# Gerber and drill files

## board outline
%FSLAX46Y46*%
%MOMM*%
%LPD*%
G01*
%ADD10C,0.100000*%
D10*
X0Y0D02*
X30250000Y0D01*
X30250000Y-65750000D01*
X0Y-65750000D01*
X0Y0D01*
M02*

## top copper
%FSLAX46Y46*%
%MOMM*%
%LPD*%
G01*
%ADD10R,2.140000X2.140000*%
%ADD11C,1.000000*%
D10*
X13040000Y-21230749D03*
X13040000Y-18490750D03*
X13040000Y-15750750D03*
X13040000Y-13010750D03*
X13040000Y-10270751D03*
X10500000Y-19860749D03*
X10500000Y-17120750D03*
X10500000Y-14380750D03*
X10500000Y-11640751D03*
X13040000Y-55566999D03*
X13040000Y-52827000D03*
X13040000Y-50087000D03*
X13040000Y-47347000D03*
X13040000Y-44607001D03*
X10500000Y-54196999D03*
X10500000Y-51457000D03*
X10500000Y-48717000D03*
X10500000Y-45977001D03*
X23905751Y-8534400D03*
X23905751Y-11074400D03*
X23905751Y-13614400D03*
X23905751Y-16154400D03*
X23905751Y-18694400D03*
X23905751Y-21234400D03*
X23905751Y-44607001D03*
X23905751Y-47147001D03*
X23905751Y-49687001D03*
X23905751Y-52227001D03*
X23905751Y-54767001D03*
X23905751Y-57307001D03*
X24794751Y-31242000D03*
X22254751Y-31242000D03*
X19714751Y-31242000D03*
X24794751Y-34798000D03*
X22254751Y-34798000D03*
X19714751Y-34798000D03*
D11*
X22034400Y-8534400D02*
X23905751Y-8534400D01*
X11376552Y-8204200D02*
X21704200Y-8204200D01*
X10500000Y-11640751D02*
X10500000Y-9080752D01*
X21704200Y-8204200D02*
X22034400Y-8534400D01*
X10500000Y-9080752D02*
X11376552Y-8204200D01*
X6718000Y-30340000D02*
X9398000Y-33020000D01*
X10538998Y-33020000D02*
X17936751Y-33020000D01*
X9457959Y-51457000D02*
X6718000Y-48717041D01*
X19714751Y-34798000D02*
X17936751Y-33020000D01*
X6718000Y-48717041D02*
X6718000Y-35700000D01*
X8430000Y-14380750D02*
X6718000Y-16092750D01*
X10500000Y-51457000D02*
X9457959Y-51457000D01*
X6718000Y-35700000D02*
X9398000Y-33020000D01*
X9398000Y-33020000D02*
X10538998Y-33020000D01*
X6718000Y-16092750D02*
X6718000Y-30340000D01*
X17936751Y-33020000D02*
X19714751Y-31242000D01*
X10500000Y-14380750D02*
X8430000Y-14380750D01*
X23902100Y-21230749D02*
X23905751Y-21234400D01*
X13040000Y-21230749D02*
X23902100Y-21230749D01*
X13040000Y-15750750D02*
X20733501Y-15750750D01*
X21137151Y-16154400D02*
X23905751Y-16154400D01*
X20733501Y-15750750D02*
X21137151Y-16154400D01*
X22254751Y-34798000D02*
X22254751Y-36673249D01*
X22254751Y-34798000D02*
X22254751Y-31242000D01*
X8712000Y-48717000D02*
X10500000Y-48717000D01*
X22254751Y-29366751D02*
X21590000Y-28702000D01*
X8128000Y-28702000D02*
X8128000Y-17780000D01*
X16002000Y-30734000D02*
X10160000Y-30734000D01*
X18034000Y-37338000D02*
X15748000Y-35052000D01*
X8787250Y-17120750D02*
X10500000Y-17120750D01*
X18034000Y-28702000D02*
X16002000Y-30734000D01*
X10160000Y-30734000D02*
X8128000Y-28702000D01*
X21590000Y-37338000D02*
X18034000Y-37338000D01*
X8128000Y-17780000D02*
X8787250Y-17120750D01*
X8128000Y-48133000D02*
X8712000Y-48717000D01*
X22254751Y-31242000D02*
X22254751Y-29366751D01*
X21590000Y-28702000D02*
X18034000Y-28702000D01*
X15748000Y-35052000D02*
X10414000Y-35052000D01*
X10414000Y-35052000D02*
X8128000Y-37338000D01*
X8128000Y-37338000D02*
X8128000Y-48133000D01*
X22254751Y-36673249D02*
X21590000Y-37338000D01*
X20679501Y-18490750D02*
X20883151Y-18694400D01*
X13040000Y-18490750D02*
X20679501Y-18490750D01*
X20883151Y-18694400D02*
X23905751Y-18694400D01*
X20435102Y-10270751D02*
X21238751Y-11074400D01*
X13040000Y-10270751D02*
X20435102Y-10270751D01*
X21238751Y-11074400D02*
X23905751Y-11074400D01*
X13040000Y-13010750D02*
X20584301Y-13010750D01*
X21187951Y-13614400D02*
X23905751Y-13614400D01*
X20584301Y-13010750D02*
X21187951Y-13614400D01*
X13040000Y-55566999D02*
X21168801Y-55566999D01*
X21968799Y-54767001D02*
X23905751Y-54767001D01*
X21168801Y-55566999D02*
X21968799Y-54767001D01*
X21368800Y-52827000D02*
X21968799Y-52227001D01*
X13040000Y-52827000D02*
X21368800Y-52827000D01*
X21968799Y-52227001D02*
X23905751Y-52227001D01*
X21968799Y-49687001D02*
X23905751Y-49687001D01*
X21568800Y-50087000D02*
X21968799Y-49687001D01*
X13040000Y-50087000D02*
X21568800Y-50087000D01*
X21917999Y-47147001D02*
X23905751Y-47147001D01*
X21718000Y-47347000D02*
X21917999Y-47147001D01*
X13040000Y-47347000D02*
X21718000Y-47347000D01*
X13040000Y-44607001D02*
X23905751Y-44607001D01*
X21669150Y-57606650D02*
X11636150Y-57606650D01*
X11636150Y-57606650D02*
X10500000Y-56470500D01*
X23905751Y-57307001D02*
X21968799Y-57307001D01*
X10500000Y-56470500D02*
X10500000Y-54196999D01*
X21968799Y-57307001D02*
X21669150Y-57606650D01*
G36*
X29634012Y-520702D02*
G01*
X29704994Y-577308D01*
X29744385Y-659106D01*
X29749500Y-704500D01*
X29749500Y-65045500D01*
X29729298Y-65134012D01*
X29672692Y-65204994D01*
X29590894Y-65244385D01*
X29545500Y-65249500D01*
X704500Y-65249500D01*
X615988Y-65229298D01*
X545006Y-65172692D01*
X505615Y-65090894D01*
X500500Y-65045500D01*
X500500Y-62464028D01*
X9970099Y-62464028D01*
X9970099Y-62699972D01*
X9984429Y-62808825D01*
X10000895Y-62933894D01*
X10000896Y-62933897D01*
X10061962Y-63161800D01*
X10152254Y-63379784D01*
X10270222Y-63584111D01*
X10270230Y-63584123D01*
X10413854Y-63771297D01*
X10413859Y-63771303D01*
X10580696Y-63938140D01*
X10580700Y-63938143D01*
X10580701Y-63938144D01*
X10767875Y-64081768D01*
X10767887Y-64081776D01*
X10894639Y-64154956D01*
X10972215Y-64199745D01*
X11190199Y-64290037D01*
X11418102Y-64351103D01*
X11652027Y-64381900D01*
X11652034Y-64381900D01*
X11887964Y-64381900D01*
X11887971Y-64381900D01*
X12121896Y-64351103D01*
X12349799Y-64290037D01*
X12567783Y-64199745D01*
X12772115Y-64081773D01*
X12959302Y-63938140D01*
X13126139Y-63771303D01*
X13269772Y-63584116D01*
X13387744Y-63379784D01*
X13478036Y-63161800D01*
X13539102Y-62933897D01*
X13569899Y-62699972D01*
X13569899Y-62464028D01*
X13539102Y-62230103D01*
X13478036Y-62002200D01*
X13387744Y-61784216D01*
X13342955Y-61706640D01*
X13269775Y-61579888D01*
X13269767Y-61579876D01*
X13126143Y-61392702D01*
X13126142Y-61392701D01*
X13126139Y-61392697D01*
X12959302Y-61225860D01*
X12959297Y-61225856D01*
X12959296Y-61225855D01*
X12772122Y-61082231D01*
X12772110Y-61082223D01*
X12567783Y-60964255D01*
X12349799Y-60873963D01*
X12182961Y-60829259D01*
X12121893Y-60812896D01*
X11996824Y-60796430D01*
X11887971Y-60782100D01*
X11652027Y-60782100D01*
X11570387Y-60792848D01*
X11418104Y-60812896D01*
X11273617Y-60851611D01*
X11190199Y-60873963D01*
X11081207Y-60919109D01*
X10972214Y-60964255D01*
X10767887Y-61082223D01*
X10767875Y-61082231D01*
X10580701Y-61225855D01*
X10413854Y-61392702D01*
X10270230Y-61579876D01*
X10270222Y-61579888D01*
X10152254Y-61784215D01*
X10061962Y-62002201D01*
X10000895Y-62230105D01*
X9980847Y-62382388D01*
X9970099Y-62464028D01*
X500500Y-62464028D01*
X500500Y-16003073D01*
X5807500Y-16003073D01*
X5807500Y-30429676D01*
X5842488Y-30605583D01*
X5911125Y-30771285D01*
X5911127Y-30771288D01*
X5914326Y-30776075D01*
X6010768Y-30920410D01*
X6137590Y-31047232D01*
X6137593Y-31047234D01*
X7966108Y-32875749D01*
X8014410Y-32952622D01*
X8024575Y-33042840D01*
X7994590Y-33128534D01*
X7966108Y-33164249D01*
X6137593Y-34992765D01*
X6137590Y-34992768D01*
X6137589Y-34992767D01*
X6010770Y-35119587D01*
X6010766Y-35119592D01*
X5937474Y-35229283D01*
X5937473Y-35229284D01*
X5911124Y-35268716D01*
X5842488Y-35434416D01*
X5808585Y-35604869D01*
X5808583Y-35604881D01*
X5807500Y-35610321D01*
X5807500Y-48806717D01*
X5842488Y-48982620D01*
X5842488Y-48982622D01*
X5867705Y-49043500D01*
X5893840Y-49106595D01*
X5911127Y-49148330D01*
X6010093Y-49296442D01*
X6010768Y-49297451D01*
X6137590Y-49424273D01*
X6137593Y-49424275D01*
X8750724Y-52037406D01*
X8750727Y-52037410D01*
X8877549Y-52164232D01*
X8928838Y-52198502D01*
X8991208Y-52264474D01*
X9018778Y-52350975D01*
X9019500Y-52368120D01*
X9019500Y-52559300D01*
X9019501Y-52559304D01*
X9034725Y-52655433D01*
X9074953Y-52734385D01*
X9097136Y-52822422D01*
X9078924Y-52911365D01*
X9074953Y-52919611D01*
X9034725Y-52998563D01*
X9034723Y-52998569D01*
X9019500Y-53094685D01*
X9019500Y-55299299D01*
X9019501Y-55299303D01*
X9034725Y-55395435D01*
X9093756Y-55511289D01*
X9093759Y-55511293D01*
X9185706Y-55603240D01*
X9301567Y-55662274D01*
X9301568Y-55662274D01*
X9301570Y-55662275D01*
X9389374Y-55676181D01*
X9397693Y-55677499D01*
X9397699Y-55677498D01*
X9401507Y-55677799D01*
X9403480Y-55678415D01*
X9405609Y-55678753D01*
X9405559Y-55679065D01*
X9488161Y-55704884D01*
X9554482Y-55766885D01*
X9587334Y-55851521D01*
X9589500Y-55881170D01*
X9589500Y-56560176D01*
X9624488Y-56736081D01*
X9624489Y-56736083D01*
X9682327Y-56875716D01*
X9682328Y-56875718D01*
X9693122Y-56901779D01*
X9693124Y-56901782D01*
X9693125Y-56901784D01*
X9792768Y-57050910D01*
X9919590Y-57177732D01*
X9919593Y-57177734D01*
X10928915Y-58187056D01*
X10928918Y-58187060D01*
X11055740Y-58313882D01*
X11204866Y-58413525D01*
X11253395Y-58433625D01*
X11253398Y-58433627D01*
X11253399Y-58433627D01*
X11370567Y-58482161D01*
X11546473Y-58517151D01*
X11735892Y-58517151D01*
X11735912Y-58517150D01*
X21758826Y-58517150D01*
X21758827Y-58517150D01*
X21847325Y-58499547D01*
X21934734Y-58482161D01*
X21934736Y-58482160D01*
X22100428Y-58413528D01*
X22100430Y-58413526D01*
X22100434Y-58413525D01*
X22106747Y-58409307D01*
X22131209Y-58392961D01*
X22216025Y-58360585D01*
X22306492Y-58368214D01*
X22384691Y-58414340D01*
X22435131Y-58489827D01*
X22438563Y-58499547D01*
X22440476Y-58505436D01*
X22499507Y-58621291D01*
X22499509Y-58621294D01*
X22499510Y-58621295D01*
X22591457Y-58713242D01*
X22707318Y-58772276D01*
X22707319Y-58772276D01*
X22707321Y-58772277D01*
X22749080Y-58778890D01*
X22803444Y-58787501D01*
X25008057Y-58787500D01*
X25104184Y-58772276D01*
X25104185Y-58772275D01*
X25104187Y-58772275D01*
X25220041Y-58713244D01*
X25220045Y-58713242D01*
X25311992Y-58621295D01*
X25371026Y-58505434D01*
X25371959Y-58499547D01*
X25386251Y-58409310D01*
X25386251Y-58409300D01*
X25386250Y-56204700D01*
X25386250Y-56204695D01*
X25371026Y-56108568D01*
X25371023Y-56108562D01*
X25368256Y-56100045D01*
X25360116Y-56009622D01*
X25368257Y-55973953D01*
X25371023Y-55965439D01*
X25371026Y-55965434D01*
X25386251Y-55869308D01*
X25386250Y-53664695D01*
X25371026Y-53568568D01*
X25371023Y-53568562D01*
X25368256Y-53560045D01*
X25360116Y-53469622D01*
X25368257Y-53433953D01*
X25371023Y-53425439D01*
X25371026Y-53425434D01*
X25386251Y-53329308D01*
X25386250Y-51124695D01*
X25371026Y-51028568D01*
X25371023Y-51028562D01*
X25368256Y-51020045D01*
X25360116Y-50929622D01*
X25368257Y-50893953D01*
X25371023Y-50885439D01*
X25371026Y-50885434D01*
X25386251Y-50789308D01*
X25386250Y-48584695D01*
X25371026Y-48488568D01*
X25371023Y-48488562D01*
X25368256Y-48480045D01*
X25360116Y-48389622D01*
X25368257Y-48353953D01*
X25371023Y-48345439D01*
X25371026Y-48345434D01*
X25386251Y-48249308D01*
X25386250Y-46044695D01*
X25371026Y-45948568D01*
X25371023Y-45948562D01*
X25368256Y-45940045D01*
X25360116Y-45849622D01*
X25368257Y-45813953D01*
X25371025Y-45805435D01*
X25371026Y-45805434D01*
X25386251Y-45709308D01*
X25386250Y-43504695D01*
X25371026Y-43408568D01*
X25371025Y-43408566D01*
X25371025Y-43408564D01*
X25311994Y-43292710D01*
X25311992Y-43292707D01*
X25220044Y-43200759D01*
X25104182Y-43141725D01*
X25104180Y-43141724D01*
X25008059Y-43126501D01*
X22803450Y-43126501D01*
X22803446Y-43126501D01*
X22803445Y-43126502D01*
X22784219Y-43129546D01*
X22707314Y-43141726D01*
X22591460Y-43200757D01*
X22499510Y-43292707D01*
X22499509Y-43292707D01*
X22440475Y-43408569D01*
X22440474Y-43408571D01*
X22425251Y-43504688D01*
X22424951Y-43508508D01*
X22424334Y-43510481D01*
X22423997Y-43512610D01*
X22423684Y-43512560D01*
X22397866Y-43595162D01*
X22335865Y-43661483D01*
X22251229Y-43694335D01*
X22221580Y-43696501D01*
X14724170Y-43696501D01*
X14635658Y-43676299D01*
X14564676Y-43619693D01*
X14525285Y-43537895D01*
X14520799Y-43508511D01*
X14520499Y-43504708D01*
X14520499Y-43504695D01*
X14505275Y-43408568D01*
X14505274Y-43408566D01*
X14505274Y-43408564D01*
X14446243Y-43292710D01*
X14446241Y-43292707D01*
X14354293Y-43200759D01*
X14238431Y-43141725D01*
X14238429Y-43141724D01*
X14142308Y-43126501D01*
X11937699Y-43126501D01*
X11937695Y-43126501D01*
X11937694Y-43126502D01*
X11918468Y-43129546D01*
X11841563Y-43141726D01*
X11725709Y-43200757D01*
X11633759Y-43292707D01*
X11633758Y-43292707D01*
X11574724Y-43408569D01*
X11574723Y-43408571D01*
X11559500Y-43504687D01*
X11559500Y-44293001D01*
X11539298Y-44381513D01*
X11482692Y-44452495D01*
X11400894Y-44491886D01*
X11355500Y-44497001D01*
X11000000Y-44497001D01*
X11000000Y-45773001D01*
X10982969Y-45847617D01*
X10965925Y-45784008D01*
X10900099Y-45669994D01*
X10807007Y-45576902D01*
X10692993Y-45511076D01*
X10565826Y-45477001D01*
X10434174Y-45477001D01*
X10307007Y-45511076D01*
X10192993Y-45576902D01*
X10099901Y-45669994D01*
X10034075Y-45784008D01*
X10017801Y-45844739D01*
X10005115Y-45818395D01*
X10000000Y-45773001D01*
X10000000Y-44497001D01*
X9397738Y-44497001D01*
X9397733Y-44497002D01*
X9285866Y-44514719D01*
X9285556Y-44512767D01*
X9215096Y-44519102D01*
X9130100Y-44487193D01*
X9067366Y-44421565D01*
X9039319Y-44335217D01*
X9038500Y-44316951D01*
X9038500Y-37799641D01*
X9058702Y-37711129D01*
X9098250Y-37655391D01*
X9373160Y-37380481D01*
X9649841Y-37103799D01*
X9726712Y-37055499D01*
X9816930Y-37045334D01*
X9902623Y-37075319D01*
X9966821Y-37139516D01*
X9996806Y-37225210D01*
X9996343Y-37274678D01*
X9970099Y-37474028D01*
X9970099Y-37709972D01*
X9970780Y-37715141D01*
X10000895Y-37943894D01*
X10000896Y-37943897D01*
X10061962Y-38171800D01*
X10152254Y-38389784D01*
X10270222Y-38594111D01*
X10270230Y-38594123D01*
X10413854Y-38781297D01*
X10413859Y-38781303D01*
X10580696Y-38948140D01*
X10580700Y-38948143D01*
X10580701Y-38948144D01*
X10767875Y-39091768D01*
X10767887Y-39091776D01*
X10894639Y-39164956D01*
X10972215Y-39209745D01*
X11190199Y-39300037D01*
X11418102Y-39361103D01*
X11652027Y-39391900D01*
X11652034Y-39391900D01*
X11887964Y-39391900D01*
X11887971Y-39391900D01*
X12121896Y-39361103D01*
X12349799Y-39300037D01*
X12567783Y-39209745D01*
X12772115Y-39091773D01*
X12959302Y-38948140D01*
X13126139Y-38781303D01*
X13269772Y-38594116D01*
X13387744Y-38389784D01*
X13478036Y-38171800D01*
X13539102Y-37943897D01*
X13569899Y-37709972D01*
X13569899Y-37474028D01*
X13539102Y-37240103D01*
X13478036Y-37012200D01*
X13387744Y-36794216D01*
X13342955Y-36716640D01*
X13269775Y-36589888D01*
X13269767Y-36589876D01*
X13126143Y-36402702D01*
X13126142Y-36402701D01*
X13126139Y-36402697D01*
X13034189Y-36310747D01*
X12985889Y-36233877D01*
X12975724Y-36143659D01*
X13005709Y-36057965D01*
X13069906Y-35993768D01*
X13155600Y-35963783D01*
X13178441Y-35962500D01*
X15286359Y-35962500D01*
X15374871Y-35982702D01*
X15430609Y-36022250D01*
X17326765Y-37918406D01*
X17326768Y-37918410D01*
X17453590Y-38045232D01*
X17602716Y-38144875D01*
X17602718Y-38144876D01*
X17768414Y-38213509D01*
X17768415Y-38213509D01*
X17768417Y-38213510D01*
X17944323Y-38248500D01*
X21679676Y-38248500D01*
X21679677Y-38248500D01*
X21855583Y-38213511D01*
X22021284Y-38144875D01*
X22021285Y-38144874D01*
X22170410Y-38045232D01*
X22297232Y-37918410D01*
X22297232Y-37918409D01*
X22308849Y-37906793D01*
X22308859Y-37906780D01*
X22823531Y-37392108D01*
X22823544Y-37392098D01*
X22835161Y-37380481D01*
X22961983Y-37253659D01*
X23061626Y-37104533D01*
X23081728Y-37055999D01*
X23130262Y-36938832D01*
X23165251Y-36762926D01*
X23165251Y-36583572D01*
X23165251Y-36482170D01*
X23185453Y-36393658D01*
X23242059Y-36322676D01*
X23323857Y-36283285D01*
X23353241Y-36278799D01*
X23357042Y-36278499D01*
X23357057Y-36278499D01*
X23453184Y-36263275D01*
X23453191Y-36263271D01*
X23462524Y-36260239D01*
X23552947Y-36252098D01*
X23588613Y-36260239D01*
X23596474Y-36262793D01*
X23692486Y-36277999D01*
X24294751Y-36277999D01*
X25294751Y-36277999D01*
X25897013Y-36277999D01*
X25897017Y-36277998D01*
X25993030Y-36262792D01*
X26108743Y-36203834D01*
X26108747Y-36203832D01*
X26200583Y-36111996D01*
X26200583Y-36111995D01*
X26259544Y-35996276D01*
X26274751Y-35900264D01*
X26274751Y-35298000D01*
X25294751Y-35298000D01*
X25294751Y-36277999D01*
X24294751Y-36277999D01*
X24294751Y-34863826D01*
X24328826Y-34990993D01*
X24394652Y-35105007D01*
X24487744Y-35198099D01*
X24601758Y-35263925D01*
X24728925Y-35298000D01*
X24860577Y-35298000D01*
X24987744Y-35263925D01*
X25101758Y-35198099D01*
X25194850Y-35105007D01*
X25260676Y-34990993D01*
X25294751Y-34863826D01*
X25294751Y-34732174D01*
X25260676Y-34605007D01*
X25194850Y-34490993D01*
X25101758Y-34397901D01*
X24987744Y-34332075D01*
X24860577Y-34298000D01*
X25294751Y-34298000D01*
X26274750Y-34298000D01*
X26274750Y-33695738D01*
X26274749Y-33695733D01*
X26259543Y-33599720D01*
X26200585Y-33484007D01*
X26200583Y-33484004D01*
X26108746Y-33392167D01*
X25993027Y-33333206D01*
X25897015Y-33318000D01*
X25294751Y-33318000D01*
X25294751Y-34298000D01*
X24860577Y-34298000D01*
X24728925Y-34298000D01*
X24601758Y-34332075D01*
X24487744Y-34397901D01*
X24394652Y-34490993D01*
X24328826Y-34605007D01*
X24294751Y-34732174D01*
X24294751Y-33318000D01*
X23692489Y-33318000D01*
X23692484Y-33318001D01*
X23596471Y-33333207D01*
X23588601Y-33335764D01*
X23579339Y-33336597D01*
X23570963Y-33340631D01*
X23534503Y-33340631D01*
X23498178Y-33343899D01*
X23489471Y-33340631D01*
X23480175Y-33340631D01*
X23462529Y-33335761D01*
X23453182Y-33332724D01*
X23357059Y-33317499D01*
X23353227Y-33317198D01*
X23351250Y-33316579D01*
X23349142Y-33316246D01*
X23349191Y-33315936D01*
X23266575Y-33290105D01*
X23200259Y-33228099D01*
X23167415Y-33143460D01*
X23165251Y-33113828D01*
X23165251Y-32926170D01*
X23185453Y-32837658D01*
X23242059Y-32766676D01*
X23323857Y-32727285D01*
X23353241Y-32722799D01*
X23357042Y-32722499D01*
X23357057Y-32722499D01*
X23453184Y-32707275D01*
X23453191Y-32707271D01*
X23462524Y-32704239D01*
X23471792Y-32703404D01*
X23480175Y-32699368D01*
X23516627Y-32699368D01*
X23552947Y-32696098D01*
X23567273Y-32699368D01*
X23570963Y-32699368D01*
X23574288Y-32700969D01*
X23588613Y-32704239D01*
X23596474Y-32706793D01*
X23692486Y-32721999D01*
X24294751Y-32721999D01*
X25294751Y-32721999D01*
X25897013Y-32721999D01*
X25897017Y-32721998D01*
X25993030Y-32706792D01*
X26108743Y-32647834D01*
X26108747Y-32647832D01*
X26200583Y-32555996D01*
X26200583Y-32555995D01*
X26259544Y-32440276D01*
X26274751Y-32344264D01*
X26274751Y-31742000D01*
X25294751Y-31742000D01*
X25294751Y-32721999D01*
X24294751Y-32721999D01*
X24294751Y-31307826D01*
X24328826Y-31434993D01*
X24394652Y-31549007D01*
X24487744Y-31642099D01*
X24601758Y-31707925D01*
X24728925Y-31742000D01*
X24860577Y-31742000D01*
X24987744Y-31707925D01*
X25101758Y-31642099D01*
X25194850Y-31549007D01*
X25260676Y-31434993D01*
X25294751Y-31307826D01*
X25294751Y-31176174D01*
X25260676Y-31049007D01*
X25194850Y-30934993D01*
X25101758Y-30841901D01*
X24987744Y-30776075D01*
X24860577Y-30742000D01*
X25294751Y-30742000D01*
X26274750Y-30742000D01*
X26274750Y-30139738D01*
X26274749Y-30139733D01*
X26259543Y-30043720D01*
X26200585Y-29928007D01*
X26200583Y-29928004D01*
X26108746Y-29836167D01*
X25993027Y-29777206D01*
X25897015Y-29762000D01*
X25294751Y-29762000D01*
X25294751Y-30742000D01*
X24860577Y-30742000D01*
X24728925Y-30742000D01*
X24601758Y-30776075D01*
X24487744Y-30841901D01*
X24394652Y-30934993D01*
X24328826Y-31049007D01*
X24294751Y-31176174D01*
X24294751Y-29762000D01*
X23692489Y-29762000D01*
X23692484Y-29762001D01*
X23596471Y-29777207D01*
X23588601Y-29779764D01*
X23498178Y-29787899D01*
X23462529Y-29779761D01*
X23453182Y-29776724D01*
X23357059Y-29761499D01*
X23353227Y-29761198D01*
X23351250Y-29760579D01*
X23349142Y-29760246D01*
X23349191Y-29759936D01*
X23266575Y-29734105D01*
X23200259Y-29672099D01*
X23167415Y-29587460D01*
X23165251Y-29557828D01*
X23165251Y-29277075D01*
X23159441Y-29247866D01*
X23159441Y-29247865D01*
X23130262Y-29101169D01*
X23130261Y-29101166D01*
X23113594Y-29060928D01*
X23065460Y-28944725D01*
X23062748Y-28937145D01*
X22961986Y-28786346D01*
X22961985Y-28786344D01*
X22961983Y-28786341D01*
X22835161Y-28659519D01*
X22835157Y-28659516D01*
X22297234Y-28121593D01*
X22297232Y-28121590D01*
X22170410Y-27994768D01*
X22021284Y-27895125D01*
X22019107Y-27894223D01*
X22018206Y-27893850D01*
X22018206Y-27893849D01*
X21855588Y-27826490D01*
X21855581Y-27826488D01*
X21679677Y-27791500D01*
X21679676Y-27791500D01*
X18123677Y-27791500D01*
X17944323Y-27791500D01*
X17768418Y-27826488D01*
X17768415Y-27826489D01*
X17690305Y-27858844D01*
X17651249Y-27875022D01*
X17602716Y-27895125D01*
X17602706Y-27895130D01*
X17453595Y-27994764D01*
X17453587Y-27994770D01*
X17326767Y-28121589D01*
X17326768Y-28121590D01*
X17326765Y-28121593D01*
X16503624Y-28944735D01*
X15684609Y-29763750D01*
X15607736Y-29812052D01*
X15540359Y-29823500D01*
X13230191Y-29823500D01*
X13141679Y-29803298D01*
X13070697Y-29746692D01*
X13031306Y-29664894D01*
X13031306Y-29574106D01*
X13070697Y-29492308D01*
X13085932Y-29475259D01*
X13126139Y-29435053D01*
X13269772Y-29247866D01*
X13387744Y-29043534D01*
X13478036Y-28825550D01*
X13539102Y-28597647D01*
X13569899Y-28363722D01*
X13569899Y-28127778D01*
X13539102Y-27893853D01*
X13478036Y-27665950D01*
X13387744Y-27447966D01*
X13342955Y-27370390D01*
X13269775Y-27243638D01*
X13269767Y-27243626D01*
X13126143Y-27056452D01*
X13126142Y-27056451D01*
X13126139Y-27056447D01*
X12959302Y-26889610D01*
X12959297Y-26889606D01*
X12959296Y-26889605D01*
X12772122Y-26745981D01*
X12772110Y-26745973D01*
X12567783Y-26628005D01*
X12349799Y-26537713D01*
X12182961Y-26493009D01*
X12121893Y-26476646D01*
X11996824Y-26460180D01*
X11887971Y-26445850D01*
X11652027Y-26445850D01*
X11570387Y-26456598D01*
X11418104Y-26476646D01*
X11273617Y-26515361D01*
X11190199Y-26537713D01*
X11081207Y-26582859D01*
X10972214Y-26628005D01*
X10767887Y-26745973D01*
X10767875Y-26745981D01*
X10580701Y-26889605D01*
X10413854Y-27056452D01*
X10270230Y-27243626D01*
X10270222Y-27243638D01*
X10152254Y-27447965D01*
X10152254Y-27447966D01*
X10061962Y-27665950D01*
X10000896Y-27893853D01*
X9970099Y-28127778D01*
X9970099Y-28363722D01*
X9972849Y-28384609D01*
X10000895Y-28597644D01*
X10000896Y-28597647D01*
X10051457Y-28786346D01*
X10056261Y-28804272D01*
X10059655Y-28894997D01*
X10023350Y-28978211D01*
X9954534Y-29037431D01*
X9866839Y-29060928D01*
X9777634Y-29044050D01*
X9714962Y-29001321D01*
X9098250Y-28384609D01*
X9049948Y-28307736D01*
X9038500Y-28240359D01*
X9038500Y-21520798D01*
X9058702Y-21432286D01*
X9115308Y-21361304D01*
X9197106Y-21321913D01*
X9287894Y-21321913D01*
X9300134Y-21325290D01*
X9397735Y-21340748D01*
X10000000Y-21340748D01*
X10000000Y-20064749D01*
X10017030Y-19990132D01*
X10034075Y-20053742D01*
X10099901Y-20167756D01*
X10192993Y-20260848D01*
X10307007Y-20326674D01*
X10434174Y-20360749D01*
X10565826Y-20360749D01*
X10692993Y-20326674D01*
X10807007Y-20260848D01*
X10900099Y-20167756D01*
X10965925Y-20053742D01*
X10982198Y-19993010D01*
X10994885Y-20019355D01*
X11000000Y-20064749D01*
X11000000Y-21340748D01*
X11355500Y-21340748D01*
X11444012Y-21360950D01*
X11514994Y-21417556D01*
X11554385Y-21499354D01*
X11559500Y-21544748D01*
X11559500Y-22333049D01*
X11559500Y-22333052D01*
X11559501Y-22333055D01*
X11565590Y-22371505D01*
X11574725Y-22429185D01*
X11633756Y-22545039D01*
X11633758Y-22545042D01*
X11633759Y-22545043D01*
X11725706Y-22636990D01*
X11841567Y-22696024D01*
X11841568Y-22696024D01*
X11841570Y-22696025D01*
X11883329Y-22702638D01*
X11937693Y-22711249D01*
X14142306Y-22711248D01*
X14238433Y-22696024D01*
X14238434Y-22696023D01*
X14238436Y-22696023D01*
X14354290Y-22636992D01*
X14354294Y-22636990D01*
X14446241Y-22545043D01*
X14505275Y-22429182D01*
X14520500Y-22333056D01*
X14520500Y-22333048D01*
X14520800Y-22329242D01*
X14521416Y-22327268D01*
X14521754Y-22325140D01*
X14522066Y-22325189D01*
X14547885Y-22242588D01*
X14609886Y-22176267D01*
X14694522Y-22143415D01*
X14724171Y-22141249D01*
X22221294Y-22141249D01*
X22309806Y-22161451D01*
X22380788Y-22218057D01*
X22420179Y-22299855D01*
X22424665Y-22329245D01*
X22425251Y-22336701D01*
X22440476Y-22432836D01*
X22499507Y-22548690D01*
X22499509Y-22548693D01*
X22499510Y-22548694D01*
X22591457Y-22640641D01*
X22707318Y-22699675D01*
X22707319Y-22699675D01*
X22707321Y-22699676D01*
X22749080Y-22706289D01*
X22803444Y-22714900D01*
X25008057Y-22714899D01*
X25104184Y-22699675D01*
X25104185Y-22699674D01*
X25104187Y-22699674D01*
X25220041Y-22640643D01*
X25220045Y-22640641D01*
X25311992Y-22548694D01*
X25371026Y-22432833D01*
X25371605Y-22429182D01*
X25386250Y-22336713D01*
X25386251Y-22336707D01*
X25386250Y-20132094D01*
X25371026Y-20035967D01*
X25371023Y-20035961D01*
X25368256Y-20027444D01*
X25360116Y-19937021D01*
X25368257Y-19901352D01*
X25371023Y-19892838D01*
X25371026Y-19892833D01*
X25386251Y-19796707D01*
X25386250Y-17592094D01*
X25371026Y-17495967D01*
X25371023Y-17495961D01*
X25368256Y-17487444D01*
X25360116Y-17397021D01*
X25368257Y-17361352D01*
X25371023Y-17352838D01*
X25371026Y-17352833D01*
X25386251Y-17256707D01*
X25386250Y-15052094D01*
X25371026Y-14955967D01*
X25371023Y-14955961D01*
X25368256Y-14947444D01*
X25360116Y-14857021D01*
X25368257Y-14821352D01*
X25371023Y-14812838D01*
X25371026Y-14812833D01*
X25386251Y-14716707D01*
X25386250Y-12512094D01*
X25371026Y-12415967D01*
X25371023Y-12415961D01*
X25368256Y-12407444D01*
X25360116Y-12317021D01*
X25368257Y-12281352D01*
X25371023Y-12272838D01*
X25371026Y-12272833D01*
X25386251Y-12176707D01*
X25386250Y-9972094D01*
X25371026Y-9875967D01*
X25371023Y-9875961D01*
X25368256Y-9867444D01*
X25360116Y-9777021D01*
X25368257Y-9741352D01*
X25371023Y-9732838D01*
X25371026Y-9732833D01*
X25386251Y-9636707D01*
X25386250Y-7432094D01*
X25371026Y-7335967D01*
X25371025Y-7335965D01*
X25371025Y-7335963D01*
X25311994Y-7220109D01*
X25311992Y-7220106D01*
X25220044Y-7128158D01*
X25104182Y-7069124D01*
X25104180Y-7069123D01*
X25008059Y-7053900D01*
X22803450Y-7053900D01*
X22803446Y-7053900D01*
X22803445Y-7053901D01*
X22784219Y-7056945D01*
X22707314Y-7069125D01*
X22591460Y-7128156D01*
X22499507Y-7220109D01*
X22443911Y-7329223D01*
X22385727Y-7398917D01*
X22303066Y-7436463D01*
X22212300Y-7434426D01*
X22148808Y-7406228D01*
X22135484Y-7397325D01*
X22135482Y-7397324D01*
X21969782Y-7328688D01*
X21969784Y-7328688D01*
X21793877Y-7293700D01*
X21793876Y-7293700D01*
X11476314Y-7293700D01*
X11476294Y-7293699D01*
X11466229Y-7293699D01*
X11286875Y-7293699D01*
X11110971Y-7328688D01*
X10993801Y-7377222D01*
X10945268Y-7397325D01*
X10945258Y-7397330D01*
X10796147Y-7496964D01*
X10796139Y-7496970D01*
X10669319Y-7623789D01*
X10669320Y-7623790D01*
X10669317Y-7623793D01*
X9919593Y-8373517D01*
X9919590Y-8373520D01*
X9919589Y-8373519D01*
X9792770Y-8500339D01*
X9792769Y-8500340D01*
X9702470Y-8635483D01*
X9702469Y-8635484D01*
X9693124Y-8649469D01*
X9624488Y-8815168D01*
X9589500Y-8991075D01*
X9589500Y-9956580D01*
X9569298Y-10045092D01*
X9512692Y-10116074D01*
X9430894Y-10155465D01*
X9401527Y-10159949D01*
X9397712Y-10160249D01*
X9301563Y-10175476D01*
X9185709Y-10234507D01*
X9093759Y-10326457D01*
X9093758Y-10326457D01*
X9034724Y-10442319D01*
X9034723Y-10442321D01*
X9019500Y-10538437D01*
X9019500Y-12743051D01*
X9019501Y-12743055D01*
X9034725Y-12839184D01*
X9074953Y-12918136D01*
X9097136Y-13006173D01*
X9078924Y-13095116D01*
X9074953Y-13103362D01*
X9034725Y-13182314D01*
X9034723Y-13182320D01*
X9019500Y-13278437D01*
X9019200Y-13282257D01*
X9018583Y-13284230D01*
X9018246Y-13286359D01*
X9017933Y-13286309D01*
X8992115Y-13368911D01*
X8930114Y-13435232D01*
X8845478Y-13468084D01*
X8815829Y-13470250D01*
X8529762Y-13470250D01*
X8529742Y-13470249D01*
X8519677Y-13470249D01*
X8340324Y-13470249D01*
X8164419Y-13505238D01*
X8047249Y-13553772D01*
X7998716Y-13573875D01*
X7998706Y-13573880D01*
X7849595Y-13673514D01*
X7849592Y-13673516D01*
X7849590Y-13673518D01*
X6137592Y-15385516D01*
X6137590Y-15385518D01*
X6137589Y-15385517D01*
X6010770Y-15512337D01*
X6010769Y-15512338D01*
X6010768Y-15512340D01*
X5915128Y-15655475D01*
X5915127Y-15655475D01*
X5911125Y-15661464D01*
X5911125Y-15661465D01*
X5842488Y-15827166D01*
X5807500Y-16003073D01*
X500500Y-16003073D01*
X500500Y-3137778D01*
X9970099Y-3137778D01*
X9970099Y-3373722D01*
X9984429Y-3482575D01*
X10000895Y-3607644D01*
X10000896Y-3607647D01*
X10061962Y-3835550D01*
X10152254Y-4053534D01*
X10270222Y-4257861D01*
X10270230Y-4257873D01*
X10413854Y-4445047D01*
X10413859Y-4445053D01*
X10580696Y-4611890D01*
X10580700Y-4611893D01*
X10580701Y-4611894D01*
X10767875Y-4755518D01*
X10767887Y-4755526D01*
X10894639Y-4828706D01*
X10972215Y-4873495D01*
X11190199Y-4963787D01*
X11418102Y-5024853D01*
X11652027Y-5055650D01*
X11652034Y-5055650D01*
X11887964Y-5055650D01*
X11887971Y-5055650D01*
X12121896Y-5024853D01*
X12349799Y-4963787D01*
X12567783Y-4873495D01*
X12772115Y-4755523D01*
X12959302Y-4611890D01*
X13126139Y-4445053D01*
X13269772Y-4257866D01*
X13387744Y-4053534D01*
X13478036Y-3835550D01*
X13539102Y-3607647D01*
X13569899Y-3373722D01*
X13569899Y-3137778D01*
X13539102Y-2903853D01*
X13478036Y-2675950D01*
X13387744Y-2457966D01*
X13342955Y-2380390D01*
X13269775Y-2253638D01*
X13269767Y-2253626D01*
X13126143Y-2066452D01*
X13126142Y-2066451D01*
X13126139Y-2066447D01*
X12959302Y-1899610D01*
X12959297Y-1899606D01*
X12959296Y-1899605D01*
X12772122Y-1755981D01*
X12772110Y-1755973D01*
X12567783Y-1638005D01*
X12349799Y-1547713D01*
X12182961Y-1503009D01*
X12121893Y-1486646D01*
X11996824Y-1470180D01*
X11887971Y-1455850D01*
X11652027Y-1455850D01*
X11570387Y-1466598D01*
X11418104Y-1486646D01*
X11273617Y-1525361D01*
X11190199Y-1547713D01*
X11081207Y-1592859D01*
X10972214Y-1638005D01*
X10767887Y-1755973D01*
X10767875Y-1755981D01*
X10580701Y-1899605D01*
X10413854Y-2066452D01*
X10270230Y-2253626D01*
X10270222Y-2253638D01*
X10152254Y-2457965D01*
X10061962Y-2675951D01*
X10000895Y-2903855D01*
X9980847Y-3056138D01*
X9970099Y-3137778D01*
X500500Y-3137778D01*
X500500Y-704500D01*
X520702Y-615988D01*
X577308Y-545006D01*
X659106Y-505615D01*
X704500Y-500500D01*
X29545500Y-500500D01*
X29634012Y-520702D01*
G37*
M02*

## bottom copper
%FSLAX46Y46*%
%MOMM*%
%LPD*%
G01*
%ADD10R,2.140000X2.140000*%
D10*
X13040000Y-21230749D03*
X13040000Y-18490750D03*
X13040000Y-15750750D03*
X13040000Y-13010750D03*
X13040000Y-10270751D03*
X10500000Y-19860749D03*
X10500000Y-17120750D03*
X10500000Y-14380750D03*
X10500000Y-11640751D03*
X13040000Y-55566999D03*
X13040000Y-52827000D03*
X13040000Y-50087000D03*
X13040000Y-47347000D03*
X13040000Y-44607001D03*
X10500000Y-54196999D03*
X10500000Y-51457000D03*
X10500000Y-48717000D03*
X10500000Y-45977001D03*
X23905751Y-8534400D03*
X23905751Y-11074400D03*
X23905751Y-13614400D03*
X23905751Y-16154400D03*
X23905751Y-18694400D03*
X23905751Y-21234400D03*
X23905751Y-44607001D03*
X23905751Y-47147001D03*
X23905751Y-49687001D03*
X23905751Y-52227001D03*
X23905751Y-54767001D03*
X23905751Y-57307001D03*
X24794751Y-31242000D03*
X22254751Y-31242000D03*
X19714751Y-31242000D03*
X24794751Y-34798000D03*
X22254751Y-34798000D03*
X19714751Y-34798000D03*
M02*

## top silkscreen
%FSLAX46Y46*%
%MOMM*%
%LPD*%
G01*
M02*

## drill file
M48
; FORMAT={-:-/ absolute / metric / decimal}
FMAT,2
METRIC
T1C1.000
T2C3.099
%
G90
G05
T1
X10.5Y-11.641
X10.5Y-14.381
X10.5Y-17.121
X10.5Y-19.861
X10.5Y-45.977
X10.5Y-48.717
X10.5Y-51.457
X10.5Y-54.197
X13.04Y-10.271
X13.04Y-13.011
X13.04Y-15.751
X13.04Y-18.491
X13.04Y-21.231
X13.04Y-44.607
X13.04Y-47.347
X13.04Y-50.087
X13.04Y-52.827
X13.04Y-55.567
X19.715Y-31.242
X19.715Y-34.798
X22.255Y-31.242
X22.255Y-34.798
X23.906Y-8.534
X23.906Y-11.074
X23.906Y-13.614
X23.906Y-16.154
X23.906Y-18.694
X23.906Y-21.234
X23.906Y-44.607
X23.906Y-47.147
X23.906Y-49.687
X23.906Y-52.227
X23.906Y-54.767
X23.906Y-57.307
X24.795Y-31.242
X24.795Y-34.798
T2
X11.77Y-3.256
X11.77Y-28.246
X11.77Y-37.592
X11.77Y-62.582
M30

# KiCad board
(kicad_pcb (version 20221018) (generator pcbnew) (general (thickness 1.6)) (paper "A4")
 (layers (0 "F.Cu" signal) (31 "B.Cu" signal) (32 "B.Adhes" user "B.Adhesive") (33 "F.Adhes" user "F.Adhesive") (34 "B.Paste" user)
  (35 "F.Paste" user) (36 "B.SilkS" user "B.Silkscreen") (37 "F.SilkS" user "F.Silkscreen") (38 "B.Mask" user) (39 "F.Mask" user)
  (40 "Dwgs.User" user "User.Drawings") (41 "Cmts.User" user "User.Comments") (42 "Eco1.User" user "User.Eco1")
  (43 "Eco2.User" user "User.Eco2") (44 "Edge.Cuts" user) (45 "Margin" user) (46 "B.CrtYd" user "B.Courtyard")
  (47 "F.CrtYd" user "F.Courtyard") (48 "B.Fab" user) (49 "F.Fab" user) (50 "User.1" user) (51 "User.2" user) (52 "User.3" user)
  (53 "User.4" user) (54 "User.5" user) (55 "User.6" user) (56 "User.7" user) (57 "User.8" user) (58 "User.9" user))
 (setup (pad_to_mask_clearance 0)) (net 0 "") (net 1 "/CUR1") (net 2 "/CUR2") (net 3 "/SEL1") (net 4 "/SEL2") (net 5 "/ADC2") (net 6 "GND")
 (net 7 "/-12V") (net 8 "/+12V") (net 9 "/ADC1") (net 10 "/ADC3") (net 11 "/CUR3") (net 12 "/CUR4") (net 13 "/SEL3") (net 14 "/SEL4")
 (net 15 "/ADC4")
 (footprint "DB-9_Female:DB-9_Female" (layer "B.Cu") (at 0.1 15.75075 -90)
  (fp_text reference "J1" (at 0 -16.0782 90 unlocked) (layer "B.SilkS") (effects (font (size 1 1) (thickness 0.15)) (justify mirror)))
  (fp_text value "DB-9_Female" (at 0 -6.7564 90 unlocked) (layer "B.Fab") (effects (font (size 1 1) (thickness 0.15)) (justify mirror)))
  (pad "" np_thru_hole circle (at -12.495 -11.669999 270) (size 3.0988 3.0988) (drill 3.0988) (layers "*.Cu" "*.Mask"))
  (pad "" np_thru_hole circle (at 12.495 -11.669999 270) (size 3.0988 3.0988) (drill 3.0988) (layers "*.Cu" "*.Mask"))
  (pad "1" thru_hole rect (at 5.479999 -12.94 270) (size 2.14 2.14) (drill 1) (layers "*.Cu" "*.Mask") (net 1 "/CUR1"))
  (pad "2" thru_hole rect (at 2.74 -12.94 270) (size 2.14 2.14) (drill 1) (layers "*.Cu" "*.Mask") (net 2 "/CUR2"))
  (pad "3" thru_hole rect (at 0 -12.94 270) (size 2.14 2.14) (drill 1) (layers "*.Cu" "*.Mask") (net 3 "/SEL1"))
  (pad "4" thru_hole rect (at -2.74 -12.94 270) (size 2.14 2.14) (drill 1) (layers "*.Cu" "*.Mask") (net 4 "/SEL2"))
  (pad "5" thru_hole rect (at -5.479999 -12.94 270) (size 2.14 2.14) (drill 1) (layers "*.Cu" "*.Mask") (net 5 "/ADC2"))
  (pad "6" thru_hole rect (at 4.109999 -10.4 270) (size 2.14 2.14) (drill 1) (layers "*.Cu" "*.Mask") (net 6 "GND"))
  (pad "7" thru_hole rect (at 1.37 -10.4 270) (size 2.14 2.14) (drill 1) (layers "*.Cu" "*.Mask") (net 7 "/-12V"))
  (pad "8" thru_hole rect (at -1.37 -10.4 270) (size 2.14 2.14) (drill 1) (layers "*.Cu" "*.Mask") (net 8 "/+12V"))
  (pad "9" thru_hole rect (at -4.109999 -10.4 270) (size 2.14 2.14) (drill 1) (layers "*.Cu" "*.Mask") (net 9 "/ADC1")))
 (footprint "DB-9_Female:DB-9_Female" (layer "B.Cu") (at 0.1 50.087 -90)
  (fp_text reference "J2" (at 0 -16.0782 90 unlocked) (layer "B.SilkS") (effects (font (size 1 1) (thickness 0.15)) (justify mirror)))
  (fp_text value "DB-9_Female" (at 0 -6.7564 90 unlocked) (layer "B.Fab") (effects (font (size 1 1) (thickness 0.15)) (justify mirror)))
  (pad "" np_thru_hole circle (at -12.495 -11.669999 270) (size 3.0988 3.0988) (drill 3.0988) (layers "*.Cu" "*.Mask"))
  (pad "" np_thru_hole circle (at 12.495 -11.669999 270) (size 3.0988 3.0988) (drill 3.0988) (layers "F&B.Cu" "*.Mask"))
  (pad "1" thru_hole rect (at 5.479999 -12.94 270) (size 2.14 2.14) (drill 1) (layers "*.Cu" "*.Mask") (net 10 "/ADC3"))
  (pad "2" thru_hole rect (at 2.74 -12.94 270) (size 2.14 2.14) (drill 1) (layers "*.Cu" "*.Mask") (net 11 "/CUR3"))
  (pad "3" thru_hole rect (at 0 -12.94 270) (size 2.14 2.14) (drill 1) (layers "*.Cu" "*.Mask") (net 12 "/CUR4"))
  (pad "4" thru_hole rect (at -2.74 -12.94 270) (size 2.14 2.14) (drill 1) (layers "*.Cu" "*.Mask") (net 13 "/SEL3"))
  (pad "5" thru_hole rect (at -5.479999 -12.94 270) (size 2.14 2.14) (drill 1) (layers "*.Cu" "*.Mask") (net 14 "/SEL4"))
  (pad "6" thru_hole rect (at 4.109999 -10.4 270) (size 2.14 2.14) (drill 1) (layers "*.Cu" "*.Mask") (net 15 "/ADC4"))
  (pad "7" thru_hole rect (at 1.37 -10.4 270) (size 2.14 2.14) (drill 1) (layers "*.Cu" "*.Mask") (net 8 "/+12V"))
  (pad "8" thru_hole rect (at -1.37 -10.4 270) (size 2.14 2.14) (drill 1) (layers "*.Cu" "*.Mask") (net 7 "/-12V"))
  (pad "9" thru_hole rect (at -4.109999 -10.4 270) (size 2.14 2.14) (drill 1) (layers "*.Cu" "*.Mask") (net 6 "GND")))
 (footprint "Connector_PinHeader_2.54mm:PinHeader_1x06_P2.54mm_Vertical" (layer "B.Cu") (at 23.905751 8.5344 180)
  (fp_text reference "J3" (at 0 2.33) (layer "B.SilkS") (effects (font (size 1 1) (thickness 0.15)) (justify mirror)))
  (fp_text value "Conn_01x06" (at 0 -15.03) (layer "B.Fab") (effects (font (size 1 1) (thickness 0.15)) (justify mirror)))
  (pad "1" thru_hole rect (at 0 0 180) (size 2.14 2.14) (drill 1) (layers "*.Cu" "*.Mask") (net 9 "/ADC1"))
  (pad "2" thru_hole rect (at 0 -2.54 180) (size 2.14 2.14) (drill 1) (layers "*.Cu" "*.Mask") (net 5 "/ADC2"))
  (pad "3" thru_hole rect (at 0 -5.08 180) (size 2.14 2.14) (drill 1) (layers "*.Cu" "*.Mask") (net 4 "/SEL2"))
  (pad "4" thru_hole rect (at 0 -7.62 180) (size 2.14 2.14) (drill 1) (layers "*.Cu" "*.Mask") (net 3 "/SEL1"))
  (pad "5" thru_hole rect (at 0 -10.16 180) (size 2.14 2.14) (drill 1) (layers "*.Cu" "*.Mask") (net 2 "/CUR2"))
  (pad "6" thru_hole rect (at 0 -12.7 180) (size 2.14 2.14) (drill 1) (layers "*.Cu" "*.Mask") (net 1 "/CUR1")))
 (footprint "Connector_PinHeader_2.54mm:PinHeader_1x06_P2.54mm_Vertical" (layer "B.Cu") (at 23.905751 44.607001 180)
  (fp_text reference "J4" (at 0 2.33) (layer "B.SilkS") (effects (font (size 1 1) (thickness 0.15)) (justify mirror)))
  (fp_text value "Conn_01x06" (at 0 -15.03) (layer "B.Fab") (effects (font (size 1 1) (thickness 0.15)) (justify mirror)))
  (pad "1" thru_hole rect (at 0 0 180) (size 2.14 2.14) (drill 1) (layers "*.Cu" "*.Mask") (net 14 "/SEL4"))
  (pad "2" thru_hole rect (at 0 -2.54 180) (size 2.14 2.14) (drill 1) (layers "*.Cu" "*.Mask") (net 13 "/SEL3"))
  (pad "3" thru_hole rect (at 0 -5.08 180) (size 2.14 2.14) (drill 1) (layers "*.Cu" "*.Mask") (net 12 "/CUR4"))
  (pad "4" thru_hole rect (at 0 -7.62 180) (size 2.14 2.14) (drill 1) (layers "*.Cu" "*.Mask") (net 11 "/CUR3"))
  (pad "5" thru_hole rect (at 0 -10.16 180) (size 2.14 2.14) (drill 1) (layers "*.Cu" "*.Mask") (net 10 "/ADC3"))
  (pad "6" thru_hole rect (at 0 -12.7 180) (size 2.14 2.14) (drill 1) (layers "*.Cu" "*.Mask") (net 15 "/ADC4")))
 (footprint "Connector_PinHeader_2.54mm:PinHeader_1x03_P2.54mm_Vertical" (layer "B.Cu") (at 24.794751 31.242 90)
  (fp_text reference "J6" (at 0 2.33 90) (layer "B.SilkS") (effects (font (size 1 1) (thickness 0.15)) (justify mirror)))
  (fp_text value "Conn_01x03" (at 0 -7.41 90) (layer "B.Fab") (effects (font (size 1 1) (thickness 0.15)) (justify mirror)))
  (pad "1" thru_hole rect (at 0 0 90) (size 2.14 2.14) (drill 1) (layers "*.Cu" "*.Mask") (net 6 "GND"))
  (pad "2" thru_hole rect (at 0 -2.54 90) (size 2.14 2.14) (drill 1) (layers "*.Cu" "*.Mask") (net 7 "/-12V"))
  (pad "3" thru_hole rect (at 0 -5.08 90) (size 2.14 2.14) (drill 1) (layers "*.Cu" "*.Mask") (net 8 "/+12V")))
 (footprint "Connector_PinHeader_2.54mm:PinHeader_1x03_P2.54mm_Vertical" (layer "B.Cu") (at 24.794751 34.798 90)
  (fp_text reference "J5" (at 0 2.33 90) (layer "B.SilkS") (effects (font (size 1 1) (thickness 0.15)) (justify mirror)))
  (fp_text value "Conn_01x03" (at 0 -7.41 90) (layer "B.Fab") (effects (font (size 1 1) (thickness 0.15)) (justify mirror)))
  (pad "1" thru_hole rect (at 0 0 90) (size 2.14 2.14) (drill 1) (layers "*.Cu" "*.Mask") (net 6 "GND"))
  (pad "2" thru_hole rect (at 0 -2.54 90) (size 2.14 2.14) (drill 1) (layers "*.Cu" "*.Mask") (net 7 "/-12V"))
  (pad "3" thru_hole rect (at 0 -5.08 90) (size 2.14 2.14) (drill 1) (layers "*.Cu" "*.Mask") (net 8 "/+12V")))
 (gr_rect (start 0 0) (end 30.25 65.75) (stroke (width 0.1) (type default)) (fill none) (layer "Edge.Cuts"))
 (segment (start 22.0344 8.5344) (end 23.905751 8.5344) (width 1) (layer "F.Cu") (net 9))
 (segment (start 11.376552 8.2042) (end 21.7042 8.2042) (width 1) (layer "F.Cu") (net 9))
 (segment (start 10.5 11.640751) (end 10.5 9.080752) (width 1) (layer "F.Cu") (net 9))
 (segment (start 21.7042 8.2042) (end 22.0344 8.5344) (width 1) (layer "F.Cu") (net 9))
 (segment (start 10.5 9.080752) (end 11.376552 8.2042) (width 1) (layer "F.Cu") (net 9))
 (segment (start 6.718 30.34) (end 9.398 33.02) (width 1) (layer "F.Cu") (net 8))
 (segment (start 10.538998 33.02) (end 17.936751 33.02) (width 1) (layer "F.Cu") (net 8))
 (segment (start 9.457959 51.457) (end 6.718 48.717041) (width 1) (layer "F.Cu") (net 8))
 (segment (start 19.714751 34.798) (end 17.936751 33.02) (width 1) (layer "F.Cu") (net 8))
 (segment (start 6.718 48.717041) (end 6.718 35.7) (width 1) (layer "F.Cu") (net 8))
 (segment (start 8.43 14.38075) (end 6.718 16.09275) (width 1) (layer "F.Cu") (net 8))
 (segment (start 10.5 51.457) (end 9.457959 51.457) (width 1) (layer "F.Cu") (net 8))
 (segment (start 6.718 35.7) (end 9.398 33.02) (width 1) (layer "F.Cu") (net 8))
 (segment (start 9.398 33.02) (end 10.538998 33.02) (width 1) (layer "F.Cu") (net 8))
 (segment (start 6.718 16.09275) (end 6.718 30.34) (width 1) (layer "F.Cu") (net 8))
 (segment (start 17.936751 33.02) (end 19.714751 31.242) (width 1) (layer "F.Cu") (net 8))
 (segment (start 10.5 14.38075) (end 8.43 14.38075) (width 1) (layer "F.Cu") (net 8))
 (segment (start 23.9021 21.230749) (end 23.905751 21.2344) (width 1) (layer "F.Cu") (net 1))
 (segment (start 13.04 21.230749) (end 23.9021 21.230749) (width 1) (layer "F.Cu") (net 1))
 (segment (start 13.04 15.75075) (end 20.733501 15.75075) (width 1) (layer "F.Cu") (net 3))
 (segment (start 21.137151 16.1544) (end 23.905751 16.1544) (width 1) (layer "F.Cu") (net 3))
 (segment (start 20.733501 15.75075) (end 21.137151 16.1544) (width 1) (layer "F.Cu") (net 3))
 (segment (start 22.254751 34.798) (end 22.254751 36.673249) (width 1) (layer "F.Cu") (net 7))
 (segment (start 22.254751 34.798) (end 22.254751 31.242) (width 1) (layer "F.Cu") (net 7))
 (segment (start 8.712 48.717) (end 10.5 48.717) (width 1) (layer "F.Cu") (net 7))
 (segment (start 22.254751 29.366751) (end 21.59 28.702) (width 1) (layer "F.Cu") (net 7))
 (segment (start 8.128 28.702) (end 8.128 17.78) (width 1) (layer "F.Cu") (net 7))
 (segment (start 16.002 30.734) (end 10.16 30.734) (width 1) (layer "F.Cu") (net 7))
 (segment (start 18.034 37.338) (end 15.748 35.052) (width 1) (layer "F.Cu") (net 7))
 (segment (start 8.78725 17.12075) (end 10.5 17.12075) (width 1) (layer "F.Cu") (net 7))
 (segment (start 18.034 28.702) (end 16.002 30.734) (width 1) (layer "F.Cu") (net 7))
 (segment (start 10.16 30.734) (end 8.128 28.702) (width 1) (layer "F.Cu") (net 7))
 (segment (start 21.59 37.338) (end 18.034 37.338) (width 1) (layer "F.Cu") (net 7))
 (segment (start 8.128 17.78) (end 8.78725 17.12075) (width 1) (layer "F.Cu") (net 7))
 (segment (start 8.128 48.133) (end 8.712 48.717) (width 1) (layer "F.Cu") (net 7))
 (segment (start 22.254751 31.242) (end 22.254751 29.366751) (width 1) (layer "F.Cu") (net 7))
 (segment (start 21.59 28.702) (end 18.034 28.702) (width 1) (layer "F.Cu") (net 7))
 (segment (start 15.748 35.052) (end 10.414 35.052) (width 1) (layer "F.Cu") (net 7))
 (segment (start 10.414 35.052) (end 8.128 37.338) (width 1) (layer "F.Cu") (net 7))
 (segment (start 8.128 37.338) (end 8.128 48.133) (width 1) (layer "F.Cu") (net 7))
 (segment (start 22.254751 36.673249) (end 21.59 37.338) (width 1) (layer "F.Cu") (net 7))
 (segment (start 20.679501 18.49075) (end 20.883151 18.6944) (width 1) (layer "F.Cu") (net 2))
 (segment (start 13.04 18.49075) (end 20.679501 18.49075) (width 1) (layer "F.Cu") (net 2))
 (segment (start 20.883151 18.6944) (end 23.905751 18.6944) (width 1) (layer "F.Cu") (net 2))
 (segment (start 20.435102 10.270751) (end 21.238751 11.0744) (width 1) (layer "F.Cu") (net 5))
 (segment (start 13.04 10.270751) (end 20.435102 10.270751) (width 1) (layer "F.Cu") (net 5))
 (segment (start 21.238751 11.0744) (end 23.905751 11.0744) (width 1) (layer "F.Cu") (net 5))
 (segment (start 13.04 13.01075) (end 20.584301 13.01075) (width 1) (layer "F.Cu") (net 4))
 (segment (start 21.187951 13.6144) (end 23.905751 13.6144) (width 1) (layer "F.Cu") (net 4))
 (segment (start 20.584301 13.01075) (end 21.187951 13.6144) (width 1) (layer "F.Cu") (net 4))
 (segment (start 13.04 55.566999) (end 21.168801 55.566999) (width 1) (layer "F.Cu") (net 10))
 (segment (start 21.968799 54.767001) (end 23.905751 54.767001) (width 1) (layer "F.Cu") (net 10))
 (segment (start 21.168801 55.566999) (end 21.968799 54.767001) (width 1) (layer "F.Cu") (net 10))
 (segment (start 21.3688 52.827) (end 21.968799 52.227001) (width 1) (layer "F.Cu") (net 11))
 (segment (start 13.04 52.827) (end 21.3688 52.827) (width 1) (layer "F.Cu") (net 11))
 (segment (start 21.968799 52.227001) (end 23.905751 52.227001) (width 1) (layer "F.Cu") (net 11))
 (segment (start 21.968799 49.687001) (end 23.905751 49.687001) (width 1) (layer "F.Cu") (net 12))
 (segment (start 21.5688 50.087) (end 21.968799 49.687001) (width 1) (layer "F.Cu") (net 12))
 (segment (start 13.04 50.087) (end 21.5688 50.087) (width 1) (layer "F.Cu") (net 12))
 (segment (start 21.917999 47.147001) (end 23.905751 47.147001) (width 1) (layer "F.Cu") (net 13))
 (segment (start 21.718 47.347) (end 21.917999 47.147001) (width 1) (layer "F.Cu") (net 13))
 (segment (start 13.04 47.347) (end 21.718 47.347) (width 1) (layer "F.Cu") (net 13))
 (segment (start 13.04 44.607001) (end 23.905751 44.607001) (width 1) (layer "F.Cu") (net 14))
 (segment (start 21.66915 57.60665) (end 11.63615 57.60665) (width 1) (layer "F.Cu") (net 15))
 (segment (start 11.63615 57.60665) (end 10.5 56.4705) (width 1) (layer "F.Cu") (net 15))
 (segment (start 23.905751 57.307001) (end 21.968799 57.307001) (width 1) (layer "F.Cu") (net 15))
 (segment (start 10.5 56.4705) (end 10.5 54.196999) (width 1) (layer "F.Cu") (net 15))
 (segment (start 21.968799 57.307001) (end 21.66915 57.60665) (width 1) (layer "F.Cu") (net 15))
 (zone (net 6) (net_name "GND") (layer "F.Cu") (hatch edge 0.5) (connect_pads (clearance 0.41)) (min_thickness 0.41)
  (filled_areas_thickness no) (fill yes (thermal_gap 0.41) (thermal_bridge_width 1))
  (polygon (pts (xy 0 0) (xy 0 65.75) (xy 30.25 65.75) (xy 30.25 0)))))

